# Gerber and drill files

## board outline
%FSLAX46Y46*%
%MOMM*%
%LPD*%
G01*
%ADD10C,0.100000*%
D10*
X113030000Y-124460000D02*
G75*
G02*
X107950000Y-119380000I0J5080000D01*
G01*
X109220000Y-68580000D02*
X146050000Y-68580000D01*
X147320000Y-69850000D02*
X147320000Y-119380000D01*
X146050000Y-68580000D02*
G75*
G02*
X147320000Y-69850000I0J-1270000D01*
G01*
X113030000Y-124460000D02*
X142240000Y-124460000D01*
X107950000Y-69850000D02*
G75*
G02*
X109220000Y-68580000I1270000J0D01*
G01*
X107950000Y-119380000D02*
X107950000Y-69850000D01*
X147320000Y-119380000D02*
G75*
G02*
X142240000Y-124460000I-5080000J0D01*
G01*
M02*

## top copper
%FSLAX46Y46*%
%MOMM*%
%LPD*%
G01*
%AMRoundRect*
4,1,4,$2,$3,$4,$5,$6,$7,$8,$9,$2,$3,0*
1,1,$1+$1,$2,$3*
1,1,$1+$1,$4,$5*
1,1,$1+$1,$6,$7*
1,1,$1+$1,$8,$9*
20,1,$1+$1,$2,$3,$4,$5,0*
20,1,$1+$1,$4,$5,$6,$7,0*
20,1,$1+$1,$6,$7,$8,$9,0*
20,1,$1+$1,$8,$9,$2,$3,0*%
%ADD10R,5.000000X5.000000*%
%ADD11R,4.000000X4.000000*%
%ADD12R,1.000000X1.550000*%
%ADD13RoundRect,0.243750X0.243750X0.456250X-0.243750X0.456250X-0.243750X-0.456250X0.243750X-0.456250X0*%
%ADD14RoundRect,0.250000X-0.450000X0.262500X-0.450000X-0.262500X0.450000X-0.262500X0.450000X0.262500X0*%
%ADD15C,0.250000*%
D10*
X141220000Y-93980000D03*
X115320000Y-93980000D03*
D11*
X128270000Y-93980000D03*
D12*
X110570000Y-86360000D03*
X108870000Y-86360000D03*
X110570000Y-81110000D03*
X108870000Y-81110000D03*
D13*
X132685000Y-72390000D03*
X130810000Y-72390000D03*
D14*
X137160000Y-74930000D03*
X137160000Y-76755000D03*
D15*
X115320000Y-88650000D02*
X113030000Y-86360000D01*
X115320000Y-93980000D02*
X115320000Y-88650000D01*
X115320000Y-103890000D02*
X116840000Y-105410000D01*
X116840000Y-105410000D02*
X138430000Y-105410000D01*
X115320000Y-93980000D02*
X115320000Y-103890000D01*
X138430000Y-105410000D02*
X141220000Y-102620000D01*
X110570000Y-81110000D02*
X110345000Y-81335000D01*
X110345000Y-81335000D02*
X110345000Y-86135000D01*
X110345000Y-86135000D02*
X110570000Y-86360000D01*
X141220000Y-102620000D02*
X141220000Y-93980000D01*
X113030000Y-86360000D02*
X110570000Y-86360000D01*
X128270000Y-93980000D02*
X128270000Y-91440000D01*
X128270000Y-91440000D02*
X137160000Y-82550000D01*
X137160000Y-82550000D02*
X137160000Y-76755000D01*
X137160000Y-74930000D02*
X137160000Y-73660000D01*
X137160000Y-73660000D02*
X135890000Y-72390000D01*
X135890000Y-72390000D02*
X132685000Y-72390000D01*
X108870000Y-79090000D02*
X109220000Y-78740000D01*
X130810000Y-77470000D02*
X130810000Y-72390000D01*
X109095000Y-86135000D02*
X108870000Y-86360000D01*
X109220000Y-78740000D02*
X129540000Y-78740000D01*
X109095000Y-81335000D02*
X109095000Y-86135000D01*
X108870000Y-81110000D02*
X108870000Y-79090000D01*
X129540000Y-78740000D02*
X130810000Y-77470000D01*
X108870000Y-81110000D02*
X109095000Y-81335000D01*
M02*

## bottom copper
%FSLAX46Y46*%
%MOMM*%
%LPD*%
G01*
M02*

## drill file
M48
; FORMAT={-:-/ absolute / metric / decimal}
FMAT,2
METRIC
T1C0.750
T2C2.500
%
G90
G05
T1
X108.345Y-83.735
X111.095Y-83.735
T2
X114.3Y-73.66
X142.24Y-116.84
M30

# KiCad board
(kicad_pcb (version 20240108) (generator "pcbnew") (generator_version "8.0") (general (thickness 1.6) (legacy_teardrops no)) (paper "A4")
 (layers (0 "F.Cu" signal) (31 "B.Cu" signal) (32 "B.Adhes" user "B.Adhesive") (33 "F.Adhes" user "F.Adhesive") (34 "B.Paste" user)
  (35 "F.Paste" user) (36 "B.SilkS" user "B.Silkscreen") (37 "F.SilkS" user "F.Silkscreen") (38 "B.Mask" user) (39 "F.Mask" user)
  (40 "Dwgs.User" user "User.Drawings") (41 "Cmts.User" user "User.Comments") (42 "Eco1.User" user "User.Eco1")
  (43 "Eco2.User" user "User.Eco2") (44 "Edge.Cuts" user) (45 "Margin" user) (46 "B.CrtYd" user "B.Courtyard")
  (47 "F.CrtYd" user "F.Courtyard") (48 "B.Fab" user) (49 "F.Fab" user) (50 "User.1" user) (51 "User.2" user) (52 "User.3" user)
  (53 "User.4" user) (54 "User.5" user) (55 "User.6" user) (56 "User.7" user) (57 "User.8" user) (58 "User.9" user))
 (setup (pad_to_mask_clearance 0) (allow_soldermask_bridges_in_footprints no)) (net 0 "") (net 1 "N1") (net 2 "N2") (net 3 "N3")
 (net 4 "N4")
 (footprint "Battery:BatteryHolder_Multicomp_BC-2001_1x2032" (layer "F.Cu") (at 128.27 93.98 180)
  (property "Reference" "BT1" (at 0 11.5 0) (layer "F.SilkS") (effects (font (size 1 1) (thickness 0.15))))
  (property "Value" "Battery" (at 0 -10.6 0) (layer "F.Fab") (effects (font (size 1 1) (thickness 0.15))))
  (pad "1" smd rect (at -12.95 0 180) (size 5 5) (layers "F.Cu" "F.Paste" "F.Mask") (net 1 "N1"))
  (pad "1" smd rect (at 12.95 0 180) (size 5 5) (layers "F.Cu" "F.Paste" "F.Mask") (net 1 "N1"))
  (pad "2" smd rect (at 0 0 180) (size 4 4) (layers "F.Cu" "F.Paste" "F.Mask") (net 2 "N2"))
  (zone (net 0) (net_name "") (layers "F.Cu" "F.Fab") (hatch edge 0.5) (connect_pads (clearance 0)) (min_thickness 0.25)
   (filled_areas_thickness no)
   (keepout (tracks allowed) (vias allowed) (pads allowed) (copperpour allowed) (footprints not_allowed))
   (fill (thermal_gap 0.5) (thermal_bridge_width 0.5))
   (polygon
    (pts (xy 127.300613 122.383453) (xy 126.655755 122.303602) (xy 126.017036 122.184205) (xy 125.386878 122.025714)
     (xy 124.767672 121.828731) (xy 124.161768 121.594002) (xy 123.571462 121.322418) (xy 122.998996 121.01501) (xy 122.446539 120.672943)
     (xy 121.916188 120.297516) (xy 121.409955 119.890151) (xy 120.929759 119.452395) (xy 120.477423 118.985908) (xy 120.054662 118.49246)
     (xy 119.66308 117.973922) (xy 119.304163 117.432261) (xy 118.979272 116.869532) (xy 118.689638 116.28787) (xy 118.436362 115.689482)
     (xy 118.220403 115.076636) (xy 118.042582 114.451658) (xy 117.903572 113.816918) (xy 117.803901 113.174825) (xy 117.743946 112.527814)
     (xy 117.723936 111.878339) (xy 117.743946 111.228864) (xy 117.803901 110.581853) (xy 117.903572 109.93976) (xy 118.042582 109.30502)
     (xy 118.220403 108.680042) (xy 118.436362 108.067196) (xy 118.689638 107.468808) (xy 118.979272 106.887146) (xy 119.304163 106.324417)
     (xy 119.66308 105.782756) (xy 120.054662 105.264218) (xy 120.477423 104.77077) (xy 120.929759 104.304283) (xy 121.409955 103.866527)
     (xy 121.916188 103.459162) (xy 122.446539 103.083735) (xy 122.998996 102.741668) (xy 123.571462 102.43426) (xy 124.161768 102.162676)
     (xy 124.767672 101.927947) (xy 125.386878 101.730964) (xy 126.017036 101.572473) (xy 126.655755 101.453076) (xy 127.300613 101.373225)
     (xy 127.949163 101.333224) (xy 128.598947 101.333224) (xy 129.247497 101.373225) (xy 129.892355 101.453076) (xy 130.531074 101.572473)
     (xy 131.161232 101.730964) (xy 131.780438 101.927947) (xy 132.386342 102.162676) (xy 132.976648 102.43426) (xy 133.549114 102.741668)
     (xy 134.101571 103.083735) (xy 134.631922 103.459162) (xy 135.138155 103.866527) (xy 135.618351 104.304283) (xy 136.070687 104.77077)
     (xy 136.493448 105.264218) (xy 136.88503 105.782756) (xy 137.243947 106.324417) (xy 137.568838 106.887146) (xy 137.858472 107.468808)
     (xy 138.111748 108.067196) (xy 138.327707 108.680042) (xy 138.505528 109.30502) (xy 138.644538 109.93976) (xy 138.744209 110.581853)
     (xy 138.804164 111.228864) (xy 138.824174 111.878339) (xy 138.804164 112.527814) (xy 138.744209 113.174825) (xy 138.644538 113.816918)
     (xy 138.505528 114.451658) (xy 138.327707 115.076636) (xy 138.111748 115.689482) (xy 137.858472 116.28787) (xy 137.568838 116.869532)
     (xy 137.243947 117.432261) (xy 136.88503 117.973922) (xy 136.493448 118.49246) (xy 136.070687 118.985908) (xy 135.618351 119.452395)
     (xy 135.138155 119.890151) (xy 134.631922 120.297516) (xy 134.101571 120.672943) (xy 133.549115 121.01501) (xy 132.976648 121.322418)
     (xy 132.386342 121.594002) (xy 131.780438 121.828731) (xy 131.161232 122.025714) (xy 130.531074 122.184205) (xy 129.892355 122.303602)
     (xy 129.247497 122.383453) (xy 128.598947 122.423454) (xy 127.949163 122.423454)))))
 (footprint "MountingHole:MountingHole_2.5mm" (layer "F.Cu") (at 142.24 116.84)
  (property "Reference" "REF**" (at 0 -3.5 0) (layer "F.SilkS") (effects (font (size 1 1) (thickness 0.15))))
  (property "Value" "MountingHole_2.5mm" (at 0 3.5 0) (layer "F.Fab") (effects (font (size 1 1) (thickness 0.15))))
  (pad "" np_thru_hole circle (at 0 0) (size 2.5 2.5) (drill 2.5) (layers "*.Cu" "*.Mask")))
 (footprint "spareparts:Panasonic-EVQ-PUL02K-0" (layer "F.Cu") (at 109.22 83.735 -90)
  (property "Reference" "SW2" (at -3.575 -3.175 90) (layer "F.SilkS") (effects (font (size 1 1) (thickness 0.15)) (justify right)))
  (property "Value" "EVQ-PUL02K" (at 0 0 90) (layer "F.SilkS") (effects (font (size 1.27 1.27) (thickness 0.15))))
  (pad "" np_thru_hole circle (at 0 -1.875 270) (size 0.75 0.75) (drill 0.75) (layers "*.Cu" "*.Mask"))
  (pad "" np_thru_hole circle (at 0 0.875 270) (size 0.75 0.75) (drill 0.75) (layers "*.Cu" "*.Mask"))
  (pad "1" smd rect (at 2.625 -1.35 270) (size 1.55 1) (layers "F.Cu" "F.Paste" "F.Mask") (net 1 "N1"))
  (pad "2" smd rect (at 2.625 0.35 270) (size 1.55 1) (layers "F.Cu" "F.Paste" "F.Mask") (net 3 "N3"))
  (pad "3" smd rect (at -2.625 -1.35 270) (size 1.55 1) (layers "F.Cu" "F.Paste" "F.Mask") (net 1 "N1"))
  (pad "4" smd rect (at -2.625 0.35 270) (size 1.55 1) (layers "F.Cu" "F.Paste" "F.Mask") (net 3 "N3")))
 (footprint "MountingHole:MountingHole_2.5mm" (layer "F.Cu") (at 114.3 73.66)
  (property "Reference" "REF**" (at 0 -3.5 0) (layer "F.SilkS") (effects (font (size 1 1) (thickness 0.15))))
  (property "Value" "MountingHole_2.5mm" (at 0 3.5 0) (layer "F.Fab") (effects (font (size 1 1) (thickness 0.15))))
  (pad "" np_thru_hole circle (at 0 0) (size 2.5 2.5) (drill 2.5) (layers "*.Cu" "*.Mask")))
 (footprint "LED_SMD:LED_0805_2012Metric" (layer "F.Cu") (at 131.7475 72.39 180)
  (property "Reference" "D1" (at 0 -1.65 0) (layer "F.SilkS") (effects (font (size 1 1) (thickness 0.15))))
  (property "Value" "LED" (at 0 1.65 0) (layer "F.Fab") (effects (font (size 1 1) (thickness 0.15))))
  (pad "1" smd roundrect (at -0.9375 0 180) (size 0.975 1.4) (layers "F.Cu" "F.Paste" "F.Mask") (roundrect_rratio 0.25) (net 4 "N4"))
  (pad "2" smd roundrect (at 0.9375 0 180) (size 0.975 1.4) (layers "F.Cu" "F.Paste" "F.Mask") (roundrect_rratio 0.25) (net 3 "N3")))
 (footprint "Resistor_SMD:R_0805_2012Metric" (layer "F.Cu") (at 137.16 75.8425 -90)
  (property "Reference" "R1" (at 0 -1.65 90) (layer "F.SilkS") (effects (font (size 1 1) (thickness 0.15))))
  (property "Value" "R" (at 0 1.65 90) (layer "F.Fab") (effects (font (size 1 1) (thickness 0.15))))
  (pad "1" smd roundrect (at -0.9125 0 270) (size 1.025 1.4) (layers "F.Cu" "F.Paste" "F.Mask") (roundrect_rratio 0.243902) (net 4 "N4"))
  (pad "2" smd roundrect (at 0.9125 0 270) (size 1.025 1.4) (layers "F.Cu" "F.Paste" "F.Mask") (roundrect_rratio 0.243902) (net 2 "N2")))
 (gr_arc (start 113.03 124.46) (mid 109.437898 122.972102) (end 107.95 119.38) (stroke (width 0.1) (type default)) (layer "Edge.Cuts"))
 (gr_line (start 109.22 68.58) (end 146.05 68.58) (stroke (width 0.1) (type default)) (layer "Edge.Cuts"))
 (gr_line (start 147.32 69.85) (end 147.32 119.38) (stroke (width 0.1) (type default)) (layer "Edge.Cuts"))
 (gr_arc (start 146.05 68.58) (mid 146.948026 68.951974) (end 147.32 69.85) (stroke (width 0.1) (type default)) (layer "Edge.Cuts"))
 (gr_line (start 113.03 124.46) (end 142.24 124.46) (stroke (width 0.1) (type default)) (layer "Edge.Cuts"))
 (gr_arc (start 107.95 69.85) (mid 108.321974 68.951974) (end 109.22 68.58) (stroke (width 0.1) (type default)) (layer "Edge.Cuts"))
 (gr_line (start 107.95 119.38) (end 107.95 69.85) (stroke (width 0.1) (type default)) (layer "Edge.Cuts"))
 (gr_arc (start 147.32 119.38) (mid 145.832102 122.972102) (end 142.24 124.46) (stroke (width 0.1) (type default)) (layer "Edge.Cuts"))
 (segment (start 115.32 88.65) (end 113.03 86.36) (width 0.25) (layer "F.Cu") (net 1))
 (segment (start 115.32 93.98) (end 115.32 88.65) (width 0.25) (layer "F.Cu") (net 1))
 (segment (start 115.32 103.89) (end 116.84 105.41) (width 0.25) (layer "F.Cu") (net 1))
 (segment (start 116.84 105.41) (end 138.43 105.41) (width 0.25) (layer "F.Cu") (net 1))
 (segment (start 115.32 93.98) (end 115.32 103.89) (width 0.25) (layer "F.Cu") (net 1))
 (segment (start 138.43 105.41) (end 141.22 102.62) (width 0.25) (layer "F.Cu") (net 1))
 (segment (start 110.57 81.11) (end 110.345 81.335) (width 0.25) (layer "F.Cu") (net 1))
 (segment (start 110.345 81.335) (end 110.345 86.135) (width 0.25) (layer "F.Cu") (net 1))
 (segment (start 110.345 86.135) (end 110.57 86.36) (width 0.25) (layer "F.Cu") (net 1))
 (segment (start 141.22 102.62) (end 141.22 93.98) (width 0.25) (layer "F.Cu") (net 1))
 (segment (start 113.03 86.36) (end 110.57 86.36) (width 0.25) (layer "F.Cu") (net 1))
 (segment (start 128.27 93.98) (end 128.27 91.44) (width 0.25) (layer "F.Cu") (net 2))
 (segment (start 128.27 91.44) (end 137.16 82.55) (width 0.25) (layer "F.Cu") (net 2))
 (segment (start 137.16 82.55) (end 137.16 76.755) (width 0.25) (layer "F.Cu") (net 2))
 (segment (start 137.16 74.93) (end 137.16 73.66) (width 0.25) (layer "F.Cu") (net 4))
 (segment (start 137.16 73.66) (end 135.89 72.39) (width 0.25) (layer "F.Cu") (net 4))
 (segment (start 135.89 72.39) (end 132.685 72.39) (width 0.25) (layer "F.Cu") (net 4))
 (segment (start 108.87 79.09) (end 109.22 78.74) (width 0.25) (layer "F.Cu") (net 3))
 (segment (start 130.81 77.47) (end 130.81 72.39) (width 0.25) (layer "F.Cu") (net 3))
 (segment (start 109.095 86.135) (end 108.87 86.36) (width 0.25) (layer "F.Cu") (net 3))
 (segment (start 109.22 78.74) (end 129.54 78.74) (width 0.25) (layer "F.Cu") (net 3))
 (segment (start 109.095 81.335) (end 109.095 86.135) (width 0.25) (layer "F.Cu") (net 3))
 (segment (start 108.87 81.11) (end 108.87 79.09) (width 0.25) (layer "F.Cu") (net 3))
 (segment (start 129.54 78.74) (end 130.81 77.47) (width 0.25) (layer "F.Cu") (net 3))
 (segment (start 108.87 81.11) (end 109.095 81.335) (width 0.25) (layer "F.Cu") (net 3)))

